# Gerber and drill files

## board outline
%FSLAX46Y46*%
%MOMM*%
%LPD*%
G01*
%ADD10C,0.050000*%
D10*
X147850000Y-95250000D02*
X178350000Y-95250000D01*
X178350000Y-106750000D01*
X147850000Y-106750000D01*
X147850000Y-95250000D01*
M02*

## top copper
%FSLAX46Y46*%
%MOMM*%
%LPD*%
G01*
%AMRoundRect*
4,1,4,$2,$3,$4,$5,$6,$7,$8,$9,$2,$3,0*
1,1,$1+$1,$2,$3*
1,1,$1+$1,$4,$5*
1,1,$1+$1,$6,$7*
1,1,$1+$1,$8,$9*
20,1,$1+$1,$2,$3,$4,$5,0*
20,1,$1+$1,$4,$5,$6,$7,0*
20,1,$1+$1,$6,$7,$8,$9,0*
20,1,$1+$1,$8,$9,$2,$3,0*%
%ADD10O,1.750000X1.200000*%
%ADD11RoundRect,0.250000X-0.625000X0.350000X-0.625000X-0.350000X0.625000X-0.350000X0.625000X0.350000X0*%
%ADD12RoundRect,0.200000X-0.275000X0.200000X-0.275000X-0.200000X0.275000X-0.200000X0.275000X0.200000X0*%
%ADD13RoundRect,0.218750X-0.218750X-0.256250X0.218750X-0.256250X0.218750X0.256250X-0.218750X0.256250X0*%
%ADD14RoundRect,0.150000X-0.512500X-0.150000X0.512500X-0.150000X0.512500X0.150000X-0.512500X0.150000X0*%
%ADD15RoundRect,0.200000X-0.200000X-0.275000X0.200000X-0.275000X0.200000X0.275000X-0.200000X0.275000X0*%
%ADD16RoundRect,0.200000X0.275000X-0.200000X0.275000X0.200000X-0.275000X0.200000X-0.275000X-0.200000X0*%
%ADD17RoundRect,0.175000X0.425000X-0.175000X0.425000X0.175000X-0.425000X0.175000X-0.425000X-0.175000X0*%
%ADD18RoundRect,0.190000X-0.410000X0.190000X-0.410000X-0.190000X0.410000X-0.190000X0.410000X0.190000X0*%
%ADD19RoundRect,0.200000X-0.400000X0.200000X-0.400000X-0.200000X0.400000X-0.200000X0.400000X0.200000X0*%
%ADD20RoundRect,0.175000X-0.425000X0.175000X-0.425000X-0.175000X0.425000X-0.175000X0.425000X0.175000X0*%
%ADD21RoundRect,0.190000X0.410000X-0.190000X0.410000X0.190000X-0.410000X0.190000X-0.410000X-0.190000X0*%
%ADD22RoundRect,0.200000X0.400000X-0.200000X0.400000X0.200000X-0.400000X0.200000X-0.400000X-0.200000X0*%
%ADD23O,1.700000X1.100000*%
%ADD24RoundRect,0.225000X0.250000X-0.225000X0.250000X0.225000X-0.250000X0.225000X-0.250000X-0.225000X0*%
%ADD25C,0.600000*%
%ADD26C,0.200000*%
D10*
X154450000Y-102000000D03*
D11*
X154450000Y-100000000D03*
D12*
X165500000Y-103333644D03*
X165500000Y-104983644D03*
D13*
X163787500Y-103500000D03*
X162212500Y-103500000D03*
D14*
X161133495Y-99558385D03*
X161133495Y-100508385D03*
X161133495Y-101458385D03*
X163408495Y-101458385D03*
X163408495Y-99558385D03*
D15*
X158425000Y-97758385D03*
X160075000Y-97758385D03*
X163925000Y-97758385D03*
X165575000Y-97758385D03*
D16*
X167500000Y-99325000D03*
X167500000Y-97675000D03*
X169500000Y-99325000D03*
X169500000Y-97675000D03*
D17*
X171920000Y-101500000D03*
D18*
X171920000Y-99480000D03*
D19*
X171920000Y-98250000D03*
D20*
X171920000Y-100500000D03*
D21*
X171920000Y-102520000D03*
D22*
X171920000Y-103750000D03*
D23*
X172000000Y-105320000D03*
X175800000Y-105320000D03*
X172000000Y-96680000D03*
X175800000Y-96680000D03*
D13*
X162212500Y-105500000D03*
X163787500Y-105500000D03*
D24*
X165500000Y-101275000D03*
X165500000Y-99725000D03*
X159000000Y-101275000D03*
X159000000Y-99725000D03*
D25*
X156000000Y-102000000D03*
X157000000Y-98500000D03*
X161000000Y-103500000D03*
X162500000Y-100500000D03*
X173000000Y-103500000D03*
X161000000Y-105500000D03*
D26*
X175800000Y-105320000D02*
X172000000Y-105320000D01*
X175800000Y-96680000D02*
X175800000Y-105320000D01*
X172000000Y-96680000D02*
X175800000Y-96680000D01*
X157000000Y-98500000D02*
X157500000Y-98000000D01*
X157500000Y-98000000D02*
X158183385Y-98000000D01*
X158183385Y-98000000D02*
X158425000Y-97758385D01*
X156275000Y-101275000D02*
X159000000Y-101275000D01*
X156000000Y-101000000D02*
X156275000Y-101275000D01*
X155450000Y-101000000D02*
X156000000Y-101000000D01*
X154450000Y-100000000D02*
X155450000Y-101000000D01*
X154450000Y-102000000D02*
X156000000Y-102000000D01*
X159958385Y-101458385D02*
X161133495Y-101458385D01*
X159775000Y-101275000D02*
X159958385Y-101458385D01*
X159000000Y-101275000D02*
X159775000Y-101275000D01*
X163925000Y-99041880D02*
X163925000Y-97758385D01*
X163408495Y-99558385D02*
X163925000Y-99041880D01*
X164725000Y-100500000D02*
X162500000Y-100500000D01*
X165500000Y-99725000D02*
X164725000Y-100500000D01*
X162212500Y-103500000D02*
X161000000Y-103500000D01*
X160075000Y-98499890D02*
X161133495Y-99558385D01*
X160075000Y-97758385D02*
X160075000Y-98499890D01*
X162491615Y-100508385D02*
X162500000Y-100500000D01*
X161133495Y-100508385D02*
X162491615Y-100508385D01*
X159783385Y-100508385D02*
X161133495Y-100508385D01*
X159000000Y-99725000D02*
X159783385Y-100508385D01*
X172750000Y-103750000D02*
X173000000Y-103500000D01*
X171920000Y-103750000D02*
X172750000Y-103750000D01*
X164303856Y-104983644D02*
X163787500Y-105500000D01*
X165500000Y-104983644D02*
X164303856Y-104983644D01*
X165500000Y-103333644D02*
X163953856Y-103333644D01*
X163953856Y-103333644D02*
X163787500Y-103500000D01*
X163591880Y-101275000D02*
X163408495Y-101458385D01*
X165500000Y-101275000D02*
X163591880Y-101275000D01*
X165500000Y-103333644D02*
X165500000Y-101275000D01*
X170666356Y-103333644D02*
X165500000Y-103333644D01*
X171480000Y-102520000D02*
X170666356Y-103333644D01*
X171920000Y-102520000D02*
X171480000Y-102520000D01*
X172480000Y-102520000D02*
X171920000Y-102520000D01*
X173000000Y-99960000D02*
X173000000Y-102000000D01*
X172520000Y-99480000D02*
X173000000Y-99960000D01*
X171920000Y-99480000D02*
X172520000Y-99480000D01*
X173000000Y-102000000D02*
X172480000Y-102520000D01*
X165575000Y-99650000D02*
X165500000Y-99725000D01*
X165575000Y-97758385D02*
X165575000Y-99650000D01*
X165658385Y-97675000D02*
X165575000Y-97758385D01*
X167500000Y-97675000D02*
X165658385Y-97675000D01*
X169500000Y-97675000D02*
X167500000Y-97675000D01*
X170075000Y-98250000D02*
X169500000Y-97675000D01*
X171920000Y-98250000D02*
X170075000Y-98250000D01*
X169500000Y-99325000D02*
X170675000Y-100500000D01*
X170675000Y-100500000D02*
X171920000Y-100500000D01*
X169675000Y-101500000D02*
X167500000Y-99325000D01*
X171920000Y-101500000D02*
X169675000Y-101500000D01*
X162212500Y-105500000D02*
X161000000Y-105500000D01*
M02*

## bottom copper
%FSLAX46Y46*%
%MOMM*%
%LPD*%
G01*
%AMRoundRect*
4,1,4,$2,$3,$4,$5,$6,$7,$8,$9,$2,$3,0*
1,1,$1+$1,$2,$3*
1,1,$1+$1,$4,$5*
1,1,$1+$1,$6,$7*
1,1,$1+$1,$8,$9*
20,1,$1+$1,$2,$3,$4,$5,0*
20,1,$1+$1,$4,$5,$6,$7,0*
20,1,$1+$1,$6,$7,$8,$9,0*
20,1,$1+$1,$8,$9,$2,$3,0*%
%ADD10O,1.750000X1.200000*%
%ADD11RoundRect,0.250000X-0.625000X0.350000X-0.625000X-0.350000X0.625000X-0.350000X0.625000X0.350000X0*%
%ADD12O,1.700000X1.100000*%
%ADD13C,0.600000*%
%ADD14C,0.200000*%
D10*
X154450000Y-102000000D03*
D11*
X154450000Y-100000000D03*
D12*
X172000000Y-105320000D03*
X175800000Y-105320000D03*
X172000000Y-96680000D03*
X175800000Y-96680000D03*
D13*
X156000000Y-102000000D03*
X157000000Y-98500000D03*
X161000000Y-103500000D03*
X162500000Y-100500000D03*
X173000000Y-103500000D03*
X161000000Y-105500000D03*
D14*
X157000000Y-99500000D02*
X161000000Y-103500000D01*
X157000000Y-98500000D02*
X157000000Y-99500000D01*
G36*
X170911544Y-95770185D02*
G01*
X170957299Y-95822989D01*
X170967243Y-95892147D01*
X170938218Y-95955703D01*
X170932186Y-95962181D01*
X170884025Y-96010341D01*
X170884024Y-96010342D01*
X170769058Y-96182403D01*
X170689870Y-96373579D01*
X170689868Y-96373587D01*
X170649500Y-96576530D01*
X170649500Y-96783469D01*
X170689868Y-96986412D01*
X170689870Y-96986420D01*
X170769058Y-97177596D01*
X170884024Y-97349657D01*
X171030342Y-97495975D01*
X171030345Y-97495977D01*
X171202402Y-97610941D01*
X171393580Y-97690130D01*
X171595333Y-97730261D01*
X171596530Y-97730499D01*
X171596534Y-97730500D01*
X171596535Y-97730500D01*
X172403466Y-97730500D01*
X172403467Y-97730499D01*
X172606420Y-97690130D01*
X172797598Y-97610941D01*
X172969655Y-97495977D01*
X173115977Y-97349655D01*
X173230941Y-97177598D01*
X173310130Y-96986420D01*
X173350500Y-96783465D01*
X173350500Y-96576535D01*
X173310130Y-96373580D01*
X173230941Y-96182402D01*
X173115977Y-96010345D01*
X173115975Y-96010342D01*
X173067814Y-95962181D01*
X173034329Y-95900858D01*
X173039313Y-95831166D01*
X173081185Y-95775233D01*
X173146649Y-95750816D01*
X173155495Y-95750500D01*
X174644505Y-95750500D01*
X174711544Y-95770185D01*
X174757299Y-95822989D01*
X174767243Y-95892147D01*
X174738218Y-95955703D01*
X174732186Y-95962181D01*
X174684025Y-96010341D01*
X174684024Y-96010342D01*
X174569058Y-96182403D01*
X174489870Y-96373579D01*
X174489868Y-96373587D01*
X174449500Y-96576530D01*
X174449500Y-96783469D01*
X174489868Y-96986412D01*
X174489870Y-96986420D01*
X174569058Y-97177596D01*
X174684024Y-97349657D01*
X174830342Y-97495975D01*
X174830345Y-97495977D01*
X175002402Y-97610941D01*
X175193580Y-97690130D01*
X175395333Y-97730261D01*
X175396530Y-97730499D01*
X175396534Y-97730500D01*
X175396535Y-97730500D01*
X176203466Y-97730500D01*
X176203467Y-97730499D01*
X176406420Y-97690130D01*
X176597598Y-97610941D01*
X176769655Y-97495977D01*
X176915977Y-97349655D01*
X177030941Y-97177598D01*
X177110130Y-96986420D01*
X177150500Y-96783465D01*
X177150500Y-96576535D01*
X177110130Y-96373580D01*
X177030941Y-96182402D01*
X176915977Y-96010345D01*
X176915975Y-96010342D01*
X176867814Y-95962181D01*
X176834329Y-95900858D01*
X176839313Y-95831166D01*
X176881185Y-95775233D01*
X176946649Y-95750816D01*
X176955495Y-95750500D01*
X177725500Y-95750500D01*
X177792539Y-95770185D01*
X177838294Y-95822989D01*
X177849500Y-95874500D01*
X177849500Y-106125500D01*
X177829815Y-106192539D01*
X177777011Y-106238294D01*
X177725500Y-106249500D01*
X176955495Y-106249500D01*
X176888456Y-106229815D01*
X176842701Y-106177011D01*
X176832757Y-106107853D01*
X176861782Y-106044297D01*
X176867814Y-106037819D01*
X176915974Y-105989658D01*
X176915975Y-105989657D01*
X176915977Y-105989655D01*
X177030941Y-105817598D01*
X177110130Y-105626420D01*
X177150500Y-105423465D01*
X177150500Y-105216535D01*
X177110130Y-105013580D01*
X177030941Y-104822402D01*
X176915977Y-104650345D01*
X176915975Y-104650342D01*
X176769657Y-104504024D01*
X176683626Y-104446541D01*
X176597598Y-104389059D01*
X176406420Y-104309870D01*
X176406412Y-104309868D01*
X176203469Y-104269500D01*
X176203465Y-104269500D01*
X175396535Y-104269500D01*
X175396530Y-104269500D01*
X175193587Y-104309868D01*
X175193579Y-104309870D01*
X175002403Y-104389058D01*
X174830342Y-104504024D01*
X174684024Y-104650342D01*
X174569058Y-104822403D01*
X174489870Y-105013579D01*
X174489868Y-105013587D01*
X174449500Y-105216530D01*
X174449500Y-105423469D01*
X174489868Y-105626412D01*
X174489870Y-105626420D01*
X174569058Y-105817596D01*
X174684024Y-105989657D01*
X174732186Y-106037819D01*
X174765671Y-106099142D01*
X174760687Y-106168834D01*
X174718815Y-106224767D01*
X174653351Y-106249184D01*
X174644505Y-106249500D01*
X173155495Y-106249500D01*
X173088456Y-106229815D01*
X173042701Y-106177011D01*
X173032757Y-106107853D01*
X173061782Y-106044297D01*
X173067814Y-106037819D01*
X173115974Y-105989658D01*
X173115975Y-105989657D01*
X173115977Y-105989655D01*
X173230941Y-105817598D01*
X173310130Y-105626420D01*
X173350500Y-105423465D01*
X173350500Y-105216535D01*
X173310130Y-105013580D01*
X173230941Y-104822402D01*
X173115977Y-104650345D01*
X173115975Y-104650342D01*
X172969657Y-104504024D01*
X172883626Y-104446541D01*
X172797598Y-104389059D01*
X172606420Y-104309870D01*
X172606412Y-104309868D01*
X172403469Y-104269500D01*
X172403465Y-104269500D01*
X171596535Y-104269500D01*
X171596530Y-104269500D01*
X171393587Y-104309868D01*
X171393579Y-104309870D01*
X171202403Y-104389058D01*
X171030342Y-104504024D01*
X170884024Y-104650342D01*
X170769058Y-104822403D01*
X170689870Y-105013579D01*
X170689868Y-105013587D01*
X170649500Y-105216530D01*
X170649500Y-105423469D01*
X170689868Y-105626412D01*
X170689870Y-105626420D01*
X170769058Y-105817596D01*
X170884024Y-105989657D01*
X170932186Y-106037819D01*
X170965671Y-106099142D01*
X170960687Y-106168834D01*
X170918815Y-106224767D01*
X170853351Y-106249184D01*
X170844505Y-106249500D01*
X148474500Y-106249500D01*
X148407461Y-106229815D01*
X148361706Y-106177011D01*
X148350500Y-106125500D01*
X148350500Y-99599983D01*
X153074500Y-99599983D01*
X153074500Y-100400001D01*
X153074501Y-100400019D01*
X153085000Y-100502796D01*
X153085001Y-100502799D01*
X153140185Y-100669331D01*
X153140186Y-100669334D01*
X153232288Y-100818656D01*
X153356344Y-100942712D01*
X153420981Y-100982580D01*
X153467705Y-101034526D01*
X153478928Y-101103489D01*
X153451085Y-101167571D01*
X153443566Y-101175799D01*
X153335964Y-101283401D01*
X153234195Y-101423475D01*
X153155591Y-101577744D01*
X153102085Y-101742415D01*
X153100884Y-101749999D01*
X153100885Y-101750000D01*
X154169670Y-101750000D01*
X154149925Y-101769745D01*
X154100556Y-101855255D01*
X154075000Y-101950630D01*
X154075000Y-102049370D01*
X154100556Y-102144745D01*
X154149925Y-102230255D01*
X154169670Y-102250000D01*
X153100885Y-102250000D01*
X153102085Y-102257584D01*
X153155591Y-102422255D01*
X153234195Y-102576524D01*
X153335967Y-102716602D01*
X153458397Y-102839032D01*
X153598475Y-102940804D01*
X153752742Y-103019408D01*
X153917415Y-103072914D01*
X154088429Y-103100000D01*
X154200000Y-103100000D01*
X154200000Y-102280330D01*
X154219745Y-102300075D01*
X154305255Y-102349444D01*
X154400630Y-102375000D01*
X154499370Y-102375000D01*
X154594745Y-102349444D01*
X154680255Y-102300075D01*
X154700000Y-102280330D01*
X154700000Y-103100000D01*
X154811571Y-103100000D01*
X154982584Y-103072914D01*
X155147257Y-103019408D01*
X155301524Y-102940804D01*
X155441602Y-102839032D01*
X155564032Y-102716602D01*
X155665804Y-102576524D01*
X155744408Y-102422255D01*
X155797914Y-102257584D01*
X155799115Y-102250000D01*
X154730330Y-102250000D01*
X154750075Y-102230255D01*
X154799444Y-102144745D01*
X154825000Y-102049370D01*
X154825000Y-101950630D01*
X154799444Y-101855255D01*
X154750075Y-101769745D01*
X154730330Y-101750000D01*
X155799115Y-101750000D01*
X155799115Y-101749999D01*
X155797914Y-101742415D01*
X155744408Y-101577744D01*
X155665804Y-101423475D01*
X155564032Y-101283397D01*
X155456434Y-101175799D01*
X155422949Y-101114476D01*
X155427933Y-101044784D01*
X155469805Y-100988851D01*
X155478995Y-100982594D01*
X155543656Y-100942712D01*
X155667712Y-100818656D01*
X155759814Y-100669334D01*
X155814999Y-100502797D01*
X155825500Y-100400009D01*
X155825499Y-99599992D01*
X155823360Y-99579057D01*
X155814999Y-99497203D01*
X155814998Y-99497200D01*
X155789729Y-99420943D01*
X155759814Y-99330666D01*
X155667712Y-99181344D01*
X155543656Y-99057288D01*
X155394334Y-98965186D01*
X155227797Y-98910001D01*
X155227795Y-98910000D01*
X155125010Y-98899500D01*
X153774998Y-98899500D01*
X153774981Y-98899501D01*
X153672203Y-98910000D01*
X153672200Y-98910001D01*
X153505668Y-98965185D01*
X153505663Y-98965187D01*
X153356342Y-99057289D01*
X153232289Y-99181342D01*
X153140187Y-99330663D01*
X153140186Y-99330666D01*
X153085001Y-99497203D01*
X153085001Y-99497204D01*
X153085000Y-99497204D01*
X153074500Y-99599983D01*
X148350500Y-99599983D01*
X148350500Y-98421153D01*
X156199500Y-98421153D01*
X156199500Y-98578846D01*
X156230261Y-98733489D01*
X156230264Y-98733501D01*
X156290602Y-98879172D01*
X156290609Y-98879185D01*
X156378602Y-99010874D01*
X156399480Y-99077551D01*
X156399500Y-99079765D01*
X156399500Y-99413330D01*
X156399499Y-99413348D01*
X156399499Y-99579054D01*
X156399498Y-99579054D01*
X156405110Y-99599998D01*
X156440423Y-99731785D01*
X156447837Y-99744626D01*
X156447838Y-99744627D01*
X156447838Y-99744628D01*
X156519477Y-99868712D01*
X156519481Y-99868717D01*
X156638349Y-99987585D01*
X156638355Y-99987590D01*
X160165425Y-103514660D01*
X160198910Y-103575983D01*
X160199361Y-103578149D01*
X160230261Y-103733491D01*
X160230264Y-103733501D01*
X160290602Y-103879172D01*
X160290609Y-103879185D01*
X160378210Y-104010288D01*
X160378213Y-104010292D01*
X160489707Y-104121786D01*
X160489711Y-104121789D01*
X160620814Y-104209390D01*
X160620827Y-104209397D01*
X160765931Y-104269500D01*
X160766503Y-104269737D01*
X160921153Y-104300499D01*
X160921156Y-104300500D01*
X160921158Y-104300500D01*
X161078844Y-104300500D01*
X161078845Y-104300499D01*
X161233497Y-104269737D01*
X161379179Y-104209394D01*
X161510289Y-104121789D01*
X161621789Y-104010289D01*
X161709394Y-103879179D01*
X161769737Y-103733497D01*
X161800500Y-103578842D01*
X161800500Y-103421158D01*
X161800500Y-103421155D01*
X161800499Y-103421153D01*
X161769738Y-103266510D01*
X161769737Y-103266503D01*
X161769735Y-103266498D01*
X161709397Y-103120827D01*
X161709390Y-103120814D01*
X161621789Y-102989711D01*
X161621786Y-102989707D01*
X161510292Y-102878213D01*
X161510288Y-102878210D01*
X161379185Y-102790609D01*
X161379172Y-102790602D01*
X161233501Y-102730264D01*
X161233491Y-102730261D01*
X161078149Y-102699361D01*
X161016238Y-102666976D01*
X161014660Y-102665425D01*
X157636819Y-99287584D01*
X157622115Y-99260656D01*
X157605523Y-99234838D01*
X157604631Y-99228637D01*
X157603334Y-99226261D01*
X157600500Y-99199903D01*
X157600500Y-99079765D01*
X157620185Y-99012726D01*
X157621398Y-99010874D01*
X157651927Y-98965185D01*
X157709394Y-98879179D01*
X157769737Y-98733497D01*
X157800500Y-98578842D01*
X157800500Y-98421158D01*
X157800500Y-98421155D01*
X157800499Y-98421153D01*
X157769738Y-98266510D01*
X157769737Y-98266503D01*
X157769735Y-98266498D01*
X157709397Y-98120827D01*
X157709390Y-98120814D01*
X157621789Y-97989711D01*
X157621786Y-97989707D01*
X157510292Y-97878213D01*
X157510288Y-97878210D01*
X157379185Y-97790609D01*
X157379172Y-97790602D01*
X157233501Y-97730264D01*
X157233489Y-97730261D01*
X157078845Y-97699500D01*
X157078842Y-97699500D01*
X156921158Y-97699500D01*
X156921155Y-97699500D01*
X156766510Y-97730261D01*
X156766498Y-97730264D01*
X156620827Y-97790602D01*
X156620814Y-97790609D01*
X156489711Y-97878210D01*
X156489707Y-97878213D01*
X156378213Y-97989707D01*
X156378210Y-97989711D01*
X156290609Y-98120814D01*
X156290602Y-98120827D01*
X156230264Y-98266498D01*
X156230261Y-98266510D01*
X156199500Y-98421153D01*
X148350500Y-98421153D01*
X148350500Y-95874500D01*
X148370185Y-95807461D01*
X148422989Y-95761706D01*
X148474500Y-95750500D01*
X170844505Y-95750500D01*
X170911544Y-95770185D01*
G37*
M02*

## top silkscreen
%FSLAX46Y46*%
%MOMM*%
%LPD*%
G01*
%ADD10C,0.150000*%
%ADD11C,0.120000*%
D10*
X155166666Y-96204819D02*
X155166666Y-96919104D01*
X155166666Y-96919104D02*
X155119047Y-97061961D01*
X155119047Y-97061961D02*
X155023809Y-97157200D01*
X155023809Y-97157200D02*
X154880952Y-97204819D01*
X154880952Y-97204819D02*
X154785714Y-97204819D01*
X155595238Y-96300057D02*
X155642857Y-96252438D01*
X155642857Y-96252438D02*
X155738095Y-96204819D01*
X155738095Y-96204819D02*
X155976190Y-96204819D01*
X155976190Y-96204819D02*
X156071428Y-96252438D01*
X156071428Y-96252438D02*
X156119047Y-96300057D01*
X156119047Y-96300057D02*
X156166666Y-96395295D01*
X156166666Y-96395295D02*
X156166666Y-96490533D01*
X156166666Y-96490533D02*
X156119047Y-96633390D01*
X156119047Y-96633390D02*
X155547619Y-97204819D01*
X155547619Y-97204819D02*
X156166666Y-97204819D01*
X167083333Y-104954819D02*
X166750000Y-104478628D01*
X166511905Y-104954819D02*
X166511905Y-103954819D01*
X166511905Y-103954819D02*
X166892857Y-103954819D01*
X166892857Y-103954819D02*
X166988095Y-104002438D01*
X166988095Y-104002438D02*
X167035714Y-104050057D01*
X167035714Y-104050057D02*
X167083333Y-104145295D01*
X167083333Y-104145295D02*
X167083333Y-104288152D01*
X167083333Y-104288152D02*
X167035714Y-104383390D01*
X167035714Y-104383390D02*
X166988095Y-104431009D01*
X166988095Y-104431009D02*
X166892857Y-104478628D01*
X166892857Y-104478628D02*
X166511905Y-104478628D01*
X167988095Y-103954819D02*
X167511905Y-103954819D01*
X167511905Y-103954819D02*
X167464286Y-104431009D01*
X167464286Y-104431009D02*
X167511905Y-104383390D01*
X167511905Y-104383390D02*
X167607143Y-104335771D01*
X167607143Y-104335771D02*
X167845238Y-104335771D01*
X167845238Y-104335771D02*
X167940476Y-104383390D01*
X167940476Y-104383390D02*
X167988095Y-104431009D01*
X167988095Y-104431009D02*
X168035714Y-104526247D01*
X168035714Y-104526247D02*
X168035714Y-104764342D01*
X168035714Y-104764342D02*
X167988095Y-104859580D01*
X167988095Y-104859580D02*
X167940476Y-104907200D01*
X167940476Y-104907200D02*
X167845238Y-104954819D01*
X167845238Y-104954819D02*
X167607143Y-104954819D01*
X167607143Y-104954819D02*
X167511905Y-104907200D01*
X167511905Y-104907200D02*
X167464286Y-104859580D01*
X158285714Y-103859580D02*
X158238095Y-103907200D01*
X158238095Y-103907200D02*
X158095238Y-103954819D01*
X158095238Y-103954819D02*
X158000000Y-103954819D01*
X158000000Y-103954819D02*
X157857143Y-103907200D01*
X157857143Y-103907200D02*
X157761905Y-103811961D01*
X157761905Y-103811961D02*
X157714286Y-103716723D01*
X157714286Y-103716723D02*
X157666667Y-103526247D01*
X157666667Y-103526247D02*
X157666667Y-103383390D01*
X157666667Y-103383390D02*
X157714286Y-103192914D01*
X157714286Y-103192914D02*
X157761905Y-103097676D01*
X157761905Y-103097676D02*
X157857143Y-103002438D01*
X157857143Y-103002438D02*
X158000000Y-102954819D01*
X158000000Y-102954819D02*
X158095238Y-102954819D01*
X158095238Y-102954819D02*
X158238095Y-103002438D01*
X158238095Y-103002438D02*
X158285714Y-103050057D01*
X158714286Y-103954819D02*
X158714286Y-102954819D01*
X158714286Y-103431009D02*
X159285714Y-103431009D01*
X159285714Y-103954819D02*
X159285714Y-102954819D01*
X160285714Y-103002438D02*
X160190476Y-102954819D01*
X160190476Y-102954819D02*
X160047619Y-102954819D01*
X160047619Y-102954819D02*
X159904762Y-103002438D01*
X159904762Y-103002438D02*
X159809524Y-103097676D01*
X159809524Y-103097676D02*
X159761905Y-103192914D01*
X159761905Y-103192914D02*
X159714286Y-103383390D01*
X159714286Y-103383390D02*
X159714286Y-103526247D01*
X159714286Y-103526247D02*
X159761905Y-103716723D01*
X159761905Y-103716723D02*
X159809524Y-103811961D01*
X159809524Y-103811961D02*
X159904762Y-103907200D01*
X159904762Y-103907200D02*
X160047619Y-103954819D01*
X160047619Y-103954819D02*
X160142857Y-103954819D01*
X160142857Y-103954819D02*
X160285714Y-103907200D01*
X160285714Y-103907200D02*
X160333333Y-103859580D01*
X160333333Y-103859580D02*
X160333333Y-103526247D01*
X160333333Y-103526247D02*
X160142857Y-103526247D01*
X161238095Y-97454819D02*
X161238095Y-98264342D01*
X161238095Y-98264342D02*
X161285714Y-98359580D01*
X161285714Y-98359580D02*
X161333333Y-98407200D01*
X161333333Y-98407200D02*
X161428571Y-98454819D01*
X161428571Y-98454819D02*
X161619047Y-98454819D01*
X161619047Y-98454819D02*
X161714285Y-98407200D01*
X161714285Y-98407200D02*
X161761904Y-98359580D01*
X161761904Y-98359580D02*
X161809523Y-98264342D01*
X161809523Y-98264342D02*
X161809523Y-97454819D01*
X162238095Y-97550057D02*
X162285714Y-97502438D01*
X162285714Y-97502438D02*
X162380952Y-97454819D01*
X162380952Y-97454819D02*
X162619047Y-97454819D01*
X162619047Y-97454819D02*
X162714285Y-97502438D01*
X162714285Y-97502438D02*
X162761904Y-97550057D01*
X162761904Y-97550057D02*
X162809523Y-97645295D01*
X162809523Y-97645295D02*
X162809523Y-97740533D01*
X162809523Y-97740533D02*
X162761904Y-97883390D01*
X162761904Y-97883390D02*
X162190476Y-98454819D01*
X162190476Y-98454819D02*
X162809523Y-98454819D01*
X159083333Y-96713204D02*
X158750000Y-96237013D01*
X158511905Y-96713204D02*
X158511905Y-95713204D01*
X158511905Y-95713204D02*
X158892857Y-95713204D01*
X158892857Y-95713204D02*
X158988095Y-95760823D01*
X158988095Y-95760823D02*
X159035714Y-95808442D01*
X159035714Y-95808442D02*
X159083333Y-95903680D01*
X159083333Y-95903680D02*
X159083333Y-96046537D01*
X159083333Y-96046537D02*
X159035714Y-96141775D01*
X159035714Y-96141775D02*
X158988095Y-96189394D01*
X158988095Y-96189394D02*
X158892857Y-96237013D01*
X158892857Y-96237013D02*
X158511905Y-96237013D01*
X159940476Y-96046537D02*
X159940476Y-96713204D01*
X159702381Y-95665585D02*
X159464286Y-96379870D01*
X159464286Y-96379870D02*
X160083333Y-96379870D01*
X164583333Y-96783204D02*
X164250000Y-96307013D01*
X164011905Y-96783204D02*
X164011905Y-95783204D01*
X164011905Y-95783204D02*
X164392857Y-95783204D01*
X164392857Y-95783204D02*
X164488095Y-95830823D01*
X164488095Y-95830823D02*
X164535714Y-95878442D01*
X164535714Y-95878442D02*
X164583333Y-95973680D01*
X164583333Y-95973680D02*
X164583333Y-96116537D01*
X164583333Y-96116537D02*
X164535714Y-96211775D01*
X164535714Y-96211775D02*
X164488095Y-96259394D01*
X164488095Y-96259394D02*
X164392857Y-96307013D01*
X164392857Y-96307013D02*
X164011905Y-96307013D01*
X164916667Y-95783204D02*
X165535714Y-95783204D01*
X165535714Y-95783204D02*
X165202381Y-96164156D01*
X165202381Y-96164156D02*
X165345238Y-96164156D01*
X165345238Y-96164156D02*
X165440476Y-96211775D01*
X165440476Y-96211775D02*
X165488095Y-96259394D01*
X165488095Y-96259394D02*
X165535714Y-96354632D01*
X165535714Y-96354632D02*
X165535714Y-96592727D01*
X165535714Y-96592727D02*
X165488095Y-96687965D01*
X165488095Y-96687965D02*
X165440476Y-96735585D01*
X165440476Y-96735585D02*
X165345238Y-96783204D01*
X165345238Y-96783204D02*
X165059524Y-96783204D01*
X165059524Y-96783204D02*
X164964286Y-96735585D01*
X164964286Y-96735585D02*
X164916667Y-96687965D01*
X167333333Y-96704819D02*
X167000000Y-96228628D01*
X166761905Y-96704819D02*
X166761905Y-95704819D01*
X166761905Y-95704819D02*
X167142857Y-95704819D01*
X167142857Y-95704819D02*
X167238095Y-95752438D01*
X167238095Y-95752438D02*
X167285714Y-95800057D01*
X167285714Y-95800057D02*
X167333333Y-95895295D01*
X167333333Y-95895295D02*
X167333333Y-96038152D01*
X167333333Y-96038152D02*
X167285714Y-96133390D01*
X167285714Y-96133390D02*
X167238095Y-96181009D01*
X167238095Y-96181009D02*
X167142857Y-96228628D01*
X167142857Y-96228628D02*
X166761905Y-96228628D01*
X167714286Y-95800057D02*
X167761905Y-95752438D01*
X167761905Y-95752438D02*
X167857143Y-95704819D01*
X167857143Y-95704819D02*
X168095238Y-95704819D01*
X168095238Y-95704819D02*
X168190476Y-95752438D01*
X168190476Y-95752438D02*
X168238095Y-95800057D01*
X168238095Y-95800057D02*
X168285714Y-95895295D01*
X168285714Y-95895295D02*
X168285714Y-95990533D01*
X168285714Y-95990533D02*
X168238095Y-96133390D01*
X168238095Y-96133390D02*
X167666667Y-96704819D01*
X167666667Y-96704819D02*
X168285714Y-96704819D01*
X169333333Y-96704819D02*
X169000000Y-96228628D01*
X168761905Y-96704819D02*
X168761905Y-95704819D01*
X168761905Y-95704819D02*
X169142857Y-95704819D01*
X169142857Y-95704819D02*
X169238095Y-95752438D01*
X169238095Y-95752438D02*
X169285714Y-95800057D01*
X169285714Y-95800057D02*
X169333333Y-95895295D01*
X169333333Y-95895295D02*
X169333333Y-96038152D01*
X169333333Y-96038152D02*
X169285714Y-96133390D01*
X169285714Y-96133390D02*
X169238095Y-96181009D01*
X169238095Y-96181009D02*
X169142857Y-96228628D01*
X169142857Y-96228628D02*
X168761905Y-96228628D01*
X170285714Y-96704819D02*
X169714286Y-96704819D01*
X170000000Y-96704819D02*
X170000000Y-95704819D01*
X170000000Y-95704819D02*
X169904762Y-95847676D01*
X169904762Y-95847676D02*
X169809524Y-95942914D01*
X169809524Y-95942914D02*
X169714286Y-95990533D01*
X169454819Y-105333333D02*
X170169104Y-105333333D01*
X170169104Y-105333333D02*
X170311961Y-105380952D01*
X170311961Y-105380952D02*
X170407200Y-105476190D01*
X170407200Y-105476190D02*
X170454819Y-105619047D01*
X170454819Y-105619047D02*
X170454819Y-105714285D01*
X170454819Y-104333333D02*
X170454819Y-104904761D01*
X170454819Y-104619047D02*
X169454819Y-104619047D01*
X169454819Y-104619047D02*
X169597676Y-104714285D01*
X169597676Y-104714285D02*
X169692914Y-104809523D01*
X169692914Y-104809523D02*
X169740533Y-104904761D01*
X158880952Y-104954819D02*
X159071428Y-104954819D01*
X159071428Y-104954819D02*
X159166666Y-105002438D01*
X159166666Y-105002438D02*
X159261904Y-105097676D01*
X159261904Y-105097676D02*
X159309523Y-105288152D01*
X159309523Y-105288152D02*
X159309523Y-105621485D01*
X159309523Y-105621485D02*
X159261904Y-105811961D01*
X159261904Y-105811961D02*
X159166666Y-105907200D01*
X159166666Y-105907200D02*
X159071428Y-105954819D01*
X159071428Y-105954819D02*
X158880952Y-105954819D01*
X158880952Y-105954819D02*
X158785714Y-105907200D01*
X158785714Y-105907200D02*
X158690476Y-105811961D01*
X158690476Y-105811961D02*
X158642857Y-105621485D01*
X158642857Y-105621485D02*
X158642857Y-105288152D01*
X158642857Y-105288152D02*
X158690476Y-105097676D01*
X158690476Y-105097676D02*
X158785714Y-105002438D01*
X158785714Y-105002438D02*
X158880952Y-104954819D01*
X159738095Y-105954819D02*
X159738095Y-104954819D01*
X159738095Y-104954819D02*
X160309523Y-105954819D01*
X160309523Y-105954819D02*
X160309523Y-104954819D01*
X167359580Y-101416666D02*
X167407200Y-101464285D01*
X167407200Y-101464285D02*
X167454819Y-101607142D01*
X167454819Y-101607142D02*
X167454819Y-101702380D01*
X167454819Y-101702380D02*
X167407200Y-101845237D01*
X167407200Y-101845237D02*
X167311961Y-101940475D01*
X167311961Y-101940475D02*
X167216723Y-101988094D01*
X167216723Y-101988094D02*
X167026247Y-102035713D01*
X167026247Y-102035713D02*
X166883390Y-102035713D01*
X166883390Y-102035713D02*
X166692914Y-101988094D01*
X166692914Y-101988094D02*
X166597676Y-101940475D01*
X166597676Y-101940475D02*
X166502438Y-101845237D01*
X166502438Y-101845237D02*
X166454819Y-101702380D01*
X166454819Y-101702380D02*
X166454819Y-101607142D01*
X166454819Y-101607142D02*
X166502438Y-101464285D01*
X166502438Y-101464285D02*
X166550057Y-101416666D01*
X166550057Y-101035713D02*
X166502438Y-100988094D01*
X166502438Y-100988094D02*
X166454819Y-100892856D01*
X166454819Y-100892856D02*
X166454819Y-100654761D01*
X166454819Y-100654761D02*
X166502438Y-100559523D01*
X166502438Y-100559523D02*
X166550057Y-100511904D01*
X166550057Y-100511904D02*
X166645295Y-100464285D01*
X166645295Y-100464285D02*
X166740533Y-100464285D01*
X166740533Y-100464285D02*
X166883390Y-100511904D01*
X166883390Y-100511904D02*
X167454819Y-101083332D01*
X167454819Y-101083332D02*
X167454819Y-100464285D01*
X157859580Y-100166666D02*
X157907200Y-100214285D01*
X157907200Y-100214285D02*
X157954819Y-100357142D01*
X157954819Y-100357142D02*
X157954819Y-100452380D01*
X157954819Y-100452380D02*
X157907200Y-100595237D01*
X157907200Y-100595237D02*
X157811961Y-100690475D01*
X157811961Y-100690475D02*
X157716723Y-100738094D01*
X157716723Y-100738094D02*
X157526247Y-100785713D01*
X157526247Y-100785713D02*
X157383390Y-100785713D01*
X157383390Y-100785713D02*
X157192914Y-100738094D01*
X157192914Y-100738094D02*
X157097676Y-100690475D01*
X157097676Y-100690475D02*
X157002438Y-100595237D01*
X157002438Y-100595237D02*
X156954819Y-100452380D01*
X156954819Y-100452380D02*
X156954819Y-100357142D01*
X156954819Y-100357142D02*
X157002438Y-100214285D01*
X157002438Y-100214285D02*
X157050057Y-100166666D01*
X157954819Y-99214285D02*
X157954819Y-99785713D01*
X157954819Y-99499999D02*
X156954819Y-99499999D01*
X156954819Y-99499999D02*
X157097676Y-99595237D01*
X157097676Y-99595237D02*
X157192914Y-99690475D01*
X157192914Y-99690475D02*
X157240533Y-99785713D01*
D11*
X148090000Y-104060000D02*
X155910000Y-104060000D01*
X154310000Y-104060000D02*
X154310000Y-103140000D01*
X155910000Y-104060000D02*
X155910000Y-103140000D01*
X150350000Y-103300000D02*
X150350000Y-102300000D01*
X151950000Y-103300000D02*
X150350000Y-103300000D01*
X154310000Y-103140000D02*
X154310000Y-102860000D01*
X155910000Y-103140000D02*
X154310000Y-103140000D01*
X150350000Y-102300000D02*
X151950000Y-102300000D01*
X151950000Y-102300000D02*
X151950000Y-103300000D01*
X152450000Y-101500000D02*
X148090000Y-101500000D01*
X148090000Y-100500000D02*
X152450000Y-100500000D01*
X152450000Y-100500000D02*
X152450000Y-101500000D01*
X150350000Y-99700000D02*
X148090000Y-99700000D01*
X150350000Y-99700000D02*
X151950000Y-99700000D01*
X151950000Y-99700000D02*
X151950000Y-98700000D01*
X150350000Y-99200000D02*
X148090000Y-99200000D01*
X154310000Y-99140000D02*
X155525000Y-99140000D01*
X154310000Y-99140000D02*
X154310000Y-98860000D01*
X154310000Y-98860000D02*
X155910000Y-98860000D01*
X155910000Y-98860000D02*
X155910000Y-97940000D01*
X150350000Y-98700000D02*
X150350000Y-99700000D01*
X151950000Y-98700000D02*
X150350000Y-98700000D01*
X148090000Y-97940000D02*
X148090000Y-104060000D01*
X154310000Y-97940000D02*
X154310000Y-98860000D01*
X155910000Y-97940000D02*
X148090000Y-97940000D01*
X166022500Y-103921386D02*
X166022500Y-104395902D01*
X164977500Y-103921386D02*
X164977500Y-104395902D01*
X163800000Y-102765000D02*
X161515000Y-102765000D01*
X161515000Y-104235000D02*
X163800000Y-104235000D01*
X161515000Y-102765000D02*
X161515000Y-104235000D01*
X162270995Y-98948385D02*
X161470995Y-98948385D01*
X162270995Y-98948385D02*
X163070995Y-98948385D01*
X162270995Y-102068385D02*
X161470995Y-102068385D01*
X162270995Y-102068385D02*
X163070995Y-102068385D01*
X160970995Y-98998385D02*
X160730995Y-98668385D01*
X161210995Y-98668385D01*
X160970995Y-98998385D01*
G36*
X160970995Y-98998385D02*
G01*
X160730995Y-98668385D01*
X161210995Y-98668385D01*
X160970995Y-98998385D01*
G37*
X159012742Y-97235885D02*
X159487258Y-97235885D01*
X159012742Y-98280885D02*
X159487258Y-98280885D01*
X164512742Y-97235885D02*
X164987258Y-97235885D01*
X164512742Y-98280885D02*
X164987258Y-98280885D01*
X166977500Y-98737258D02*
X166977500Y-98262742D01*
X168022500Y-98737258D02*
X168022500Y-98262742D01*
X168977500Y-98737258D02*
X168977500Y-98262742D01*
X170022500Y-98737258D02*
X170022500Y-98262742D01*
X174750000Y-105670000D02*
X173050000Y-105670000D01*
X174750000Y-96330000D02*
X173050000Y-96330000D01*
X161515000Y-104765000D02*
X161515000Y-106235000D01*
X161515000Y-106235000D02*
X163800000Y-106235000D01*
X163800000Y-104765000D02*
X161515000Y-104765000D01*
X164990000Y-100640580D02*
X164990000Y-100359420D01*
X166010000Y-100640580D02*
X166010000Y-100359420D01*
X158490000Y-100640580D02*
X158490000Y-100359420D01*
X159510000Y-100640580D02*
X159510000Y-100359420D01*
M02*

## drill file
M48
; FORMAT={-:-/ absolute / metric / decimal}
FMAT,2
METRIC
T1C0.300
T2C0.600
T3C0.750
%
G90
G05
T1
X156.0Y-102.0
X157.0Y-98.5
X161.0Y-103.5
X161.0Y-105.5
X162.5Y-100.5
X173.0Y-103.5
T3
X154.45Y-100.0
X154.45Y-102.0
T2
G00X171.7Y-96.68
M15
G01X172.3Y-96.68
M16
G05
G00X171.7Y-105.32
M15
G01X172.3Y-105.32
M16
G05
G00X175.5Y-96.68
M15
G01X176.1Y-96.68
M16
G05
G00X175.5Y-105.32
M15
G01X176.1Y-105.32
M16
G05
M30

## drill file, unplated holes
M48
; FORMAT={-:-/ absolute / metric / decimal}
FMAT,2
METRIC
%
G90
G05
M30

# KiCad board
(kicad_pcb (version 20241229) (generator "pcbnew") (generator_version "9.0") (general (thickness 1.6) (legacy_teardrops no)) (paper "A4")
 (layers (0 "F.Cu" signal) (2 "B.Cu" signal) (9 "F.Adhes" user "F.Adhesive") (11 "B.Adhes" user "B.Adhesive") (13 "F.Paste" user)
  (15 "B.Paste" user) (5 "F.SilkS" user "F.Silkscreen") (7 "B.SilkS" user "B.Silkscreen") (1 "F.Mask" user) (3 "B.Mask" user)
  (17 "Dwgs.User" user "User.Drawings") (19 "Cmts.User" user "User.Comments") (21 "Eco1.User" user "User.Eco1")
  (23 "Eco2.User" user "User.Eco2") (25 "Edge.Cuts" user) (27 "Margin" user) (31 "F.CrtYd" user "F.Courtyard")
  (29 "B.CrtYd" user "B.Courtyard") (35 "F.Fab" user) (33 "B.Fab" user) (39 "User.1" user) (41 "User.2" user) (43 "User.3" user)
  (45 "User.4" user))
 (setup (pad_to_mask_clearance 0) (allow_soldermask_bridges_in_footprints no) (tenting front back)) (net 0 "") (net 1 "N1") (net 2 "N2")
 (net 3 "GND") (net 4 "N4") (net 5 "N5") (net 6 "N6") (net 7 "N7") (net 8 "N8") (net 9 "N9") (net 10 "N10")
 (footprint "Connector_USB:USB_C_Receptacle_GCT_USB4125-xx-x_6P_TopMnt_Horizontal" (layer "F.Cu") (at 175 101 90)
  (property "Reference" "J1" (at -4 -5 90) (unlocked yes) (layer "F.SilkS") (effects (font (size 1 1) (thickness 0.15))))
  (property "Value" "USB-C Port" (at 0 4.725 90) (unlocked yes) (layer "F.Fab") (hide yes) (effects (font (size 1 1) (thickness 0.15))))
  (fp_line (start 4.67 -0.25) (end 4.67 -1.95) (stroke (width 0.12) (type solid)) (layer "F.SilkS"))
  (fp_line (start -4.67 -0.25) (end -4.67 -1.95) (stroke (width 0.12) (type solid)) (layer "F.SilkS"))
  (pad "A5" smd roundrect (at -0.5 -3.08 90) (size 0.7 1.2) (layers "F.Cu" "F.Mask" "F.Paste") (roundrect_rratio 0.25) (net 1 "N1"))
  (pad "A9" smd roundrect (at 1.52 -3.08 270) (size 0.76 1.2) (layers "F.Cu" "F.Mask" "F.Paste") (roundrect_rratio 0.25) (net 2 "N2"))
  (pad "A12" smd roundrect (at 2.75 -3.08 270) (size 0.8 1.2) (layers "F.Cu" "F.Mask" "F.Paste") (roundrect_rratio 0.25) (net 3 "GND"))
  (pad "B5" smd roundrect (at 0.5 -3.08 270) (size 0.7 1.2) (layers "F.Cu" "F.Mask" "F.Paste") (roundrect_rratio 0.25) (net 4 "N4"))
  (pad "B9" smd roundrect (at -1.52 -3.08 90) (size 0.76 1.2) (layers "F.Cu" "F.Mask" "F.Paste") (roundrect_rratio 0.25) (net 2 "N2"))
  (pad "B12" smd roundrect (at -2.75 -3.08 90) (size 0.8 1.2) (layers "F.Cu" "F.Mask" "F.Paste") (roundrect_rratio 0.25) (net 3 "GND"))
  (pad "S1" thru_hole oval (at -4.32 -3 90) (size 1.1 1.7) (drill oval 0.6 1.2) (layers "*.Cu" "*.Mask" "F.Paste") (remove_unused_layers no)
   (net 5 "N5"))
  (pad "S1" thru_hole oval (at -4.32 0.8 90) (size 1.1 1.7) (drill oval 0.6 1.2) (layers "*.Cu" "*.Mask" "F.Paste")
   (remove_unused_layers no) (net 5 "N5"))
  (pad "S1" thru_hole oval (at 4.32 -3 90) (size 1.1 1.7) (drill oval 0.6 1.2) (layers "*.Cu" "*.Mask" "F.Paste") (remove_unused_layers no)
   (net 5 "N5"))
  (pad "S1" thru_hole oval (at 4.32 0.8 90) (size 1.1 1.7) (drill oval 0.6 1.2) (layers "*.Cu" "*.Mask" "F.Paste") (remove_unused_layers no)
   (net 5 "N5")))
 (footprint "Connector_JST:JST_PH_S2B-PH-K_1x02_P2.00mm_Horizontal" (layer "F.Cu") (at 154.45 100 -90)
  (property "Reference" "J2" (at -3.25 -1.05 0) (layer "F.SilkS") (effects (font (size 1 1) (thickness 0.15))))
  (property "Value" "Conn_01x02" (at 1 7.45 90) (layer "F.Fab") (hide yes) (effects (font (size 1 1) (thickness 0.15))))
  (fp_line (start -2.06 6.36) (end 4.06 6.36) (stroke (width 0.12) (type solid)) (layer "F.SilkS"))
  (fp_line (start 0.5 6.36) (end 0.5 2) (stroke (width 0.12) (type solid)) (layer "F.SilkS"))
  (fp_line (start 4.06 6.36) (end 4.06 -1.46) (stroke (width 0.12) (type solid)) (layer "F.SilkS"))
  (fp_line (start -1.3 4.1) (end -0.3 4.1) (stroke (width 0.12) (type solid)) (layer "F.SilkS"))
  (fp_line (start -0.8 4.1) (end -0.8 6.36) (stroke (width 0.12) (type solid)) (layer "F.SilkS"))
  (fp_line (start -0.3 4.1) (end -0.3 6.36) (stroke (width 0.12) (type solid)) (layer "F.SilkS"))
  (fp_line (start -0.3 4.1) (end -0.3 2.5) (stroke (width 0.12) (type solid)) (layer "F.SilkS"))
  (fp_line (start 2.3 4.1) (end 2.3 2.5) (stroke (width 0.12) (type solid)) (layer "F.SilkS"))
  (fp_line (start 3.3 4.1) (end 2.3 4.1) (stroke (width 0.12) (type solid)) (layer "F.SilkS"))
  (fp_line (start -1.3 2.5) (end -1.3 4.1) (stroke (width 0.12) (type solid)) (layer "F.SilkS"))
  (fp_line (start -0.3 2.5) (end -1.3 2.5) (stroke (width 0.12) (type solid)) (layer "F.SilkS"))
  (fp_line (start 2.3 2.5) (end 3.3 2.5) (stroke (width 0.12) (type solid)) (layer "F.SilkS"))
  (fp_line (start 3.3 2.5) (end 3.3 4.1) (stroke (width 0.12) (type solid)) (layer "F.SilkS"))
  (fp_line (start 0.5 2) (end 1.5 2) (stroke (width 0.12) (type solid)) (layer "F.SilkS"))
  (fp_line (start 1.5 2) (end 1.5 6.36) (stroke (width 0.12) (type solid)) (layer "F.SilkS"))
  (fp_line (start -2.06 0.14) (end -1.14 0.14) (stroke (width 0.12) (type solid)) (layer "F.SilkS"))
  (fp_line (start -1.14 0.14) (end -1.14 -1.46) (stroke (width 0.12) (type solid)) (layer "F.SilkS"))
  (fp_line (start -0.86 0.14) (end -1.14 0.14) (stroke (width 0.12) (type solid)) (layer "F.SilkS"))
  (fp_line (start -0.86 0.14) (end -0.86 -1.075) (stroke (width 0.12) (type solid)) (layer "F.SilkS"))
  (fp_line (start 3.14 0.14) (end 2.86 0.14) (stroke (width 0.12) (type solid)) (layer "F.SilkS"))
  (fp_line (start 4.06 0.14) (end 3.14 0.14) (stroke (width 0.12) (type solid)) (layer "F.SilkS"))
  (fp_line (start -2.06 -1.46) (end -2.06 6.36) (stroke (width 0.12) (type solid)) (layer "F.SilkS"))
  (fp_line (start -1.14 -1.46) (end -2.06 -1.46) (stroke (width 0.12) (type solid)) (layer "F.SilkS"))
  (fp_line (start 3.14 -1.46) (end 3.14 0.14) (stroke (width 0.12) (type solid)) (layer "F.SilkS"))
  (fp_line (start 4.06 -1.46) (end 3.14 -1.46) (stroke (width 0.12) (type solid)) (layer "F.SilkS"))
  (pad "1" thru_hole roundrect (at 0 0 270) (size 1.2 1.75) (drill 0.75) (layers "*.Cu" "*.Mask") (remove_unused_layers no)
   (roundrect_rratio 0.208333) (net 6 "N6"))
  (pad "2" thru_hole oval (at 2 0 270) (size 1.2 1.75) (drill 0.75) (layers "*.Cu" "*.Mask") (remove_unused_layers no) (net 3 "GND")))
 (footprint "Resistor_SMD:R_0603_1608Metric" (layer "F.Cu") (at 164.75 97.758385)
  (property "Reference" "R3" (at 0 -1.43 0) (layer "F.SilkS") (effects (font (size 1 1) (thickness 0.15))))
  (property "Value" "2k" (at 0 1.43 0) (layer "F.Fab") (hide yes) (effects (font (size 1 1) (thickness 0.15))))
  (fp_line (start -0.237258 -0.5225) (end 0.237258 -0.5225) (stroke (width 0.12) (type solid)) (layer "F.SilkS"))
  (fp_line (start -0.237258 0.5225) (end 0.237258 0.5225) (stroke (width 0.12) (type solid)) (layer "F.SilkS"))
  (pad "1" smd roundrect (at -0.825 0) (size 0.8 0.95) (layers "F.Cu" "F.Mask" "F.Paste") (roundrect_rratio 0.25) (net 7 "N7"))
  (pad "2" smd roundrect (at 0.825 0) (size 0.8 0.95) (layers "F.Cu" "F.Mask" "F.Paste") (roundrect_rratio 0.25) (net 3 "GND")))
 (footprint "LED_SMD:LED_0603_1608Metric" (layer "F.Cu") (at 163 103.5)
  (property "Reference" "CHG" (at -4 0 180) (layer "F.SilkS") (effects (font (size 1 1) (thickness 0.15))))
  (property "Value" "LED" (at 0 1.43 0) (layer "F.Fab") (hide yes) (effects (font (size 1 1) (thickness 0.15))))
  (fp_line (start -1.485 -0.735) (end -1.485 0.735) (stroke (width 0.12) (type solid)) (layer "F.SilkS"))
  (fp_line (start -1.485 0.735) (end 0.8 0.735) (stroke (width 0.12) (type solid)) (layer "F.SilkS"))
  (fp_line (start 0.8 -0.735) (end -1.485 -0.735) (stroke (width 0.12) (type solid)) (layer "F.SilkS"))
  (pad "1" smd roundrect (at -0.7875 0) (size 0.875 0.95) (layers "F.Cu" "F.Mask" "F.Paste") (roundrect_rratio 0.25) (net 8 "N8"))
  (pad "2" smd roundrect (at 0.7875 0) (size 0.875 0.95) (layers "F.Cu" "F.Mask" "F.Paste") (roundrect_rratio 0.25) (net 2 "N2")))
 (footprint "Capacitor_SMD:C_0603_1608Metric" (layer "F.Cu") (at 165.5 100.5 90)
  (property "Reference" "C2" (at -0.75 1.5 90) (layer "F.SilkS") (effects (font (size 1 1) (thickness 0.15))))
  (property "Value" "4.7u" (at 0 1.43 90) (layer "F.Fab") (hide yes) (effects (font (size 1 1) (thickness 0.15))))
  (fp_line (start -0.14058 -0.51) (end 0.14058 -0.51) (stroke (width 0.12) (type solid)) (layer "F.SilkS"))
  (fp_line (start -0.14058 0.51) (end 0.14058 0.51) (stroke (width 0.12) (type solid)) (layer "F.SilkS"))
  (pad "1" smd roundrect (at -0.775 0 90) (size 0.9 0.95) (layers "F.Cu" "F.Mask" "F.Paste") (roundrect_rratio 0.25) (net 2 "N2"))
  (pad "2" smd roundrect (at 0.775 0 90) (size 0.9 0.95) (layers "F.Cu" "F.Mask" "F.Paste") (roundrect_rratio 0.25) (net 3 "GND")))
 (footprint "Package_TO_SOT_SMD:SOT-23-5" (layer "F.Cu") (at 162.270995 100.508385)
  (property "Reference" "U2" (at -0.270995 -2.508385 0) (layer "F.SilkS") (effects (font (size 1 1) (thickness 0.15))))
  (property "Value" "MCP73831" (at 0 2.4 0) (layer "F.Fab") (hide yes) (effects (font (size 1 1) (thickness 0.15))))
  (fp_line (start 0 -1.56) (end -0.8 -1.56) (stroke (width 0.12) (type solid)) (layer "F.SilkS"))
  (fp_line (start 0 -1.56) (end 0.8 -1.56) (stroke (width 0.12) (type solid)) (layer "F.SilkS"))
  (fp_line (start 0 1.56) (end -0.8 1.56) (stroke (width 0.12) (type solid)) (layer "F.SilkS"))
  (fp_line (start 0 1.56) (end 0.8 1.56) (stroke (width 0.12) (type solid)) (layer "F.SilkS"))
  (fp_poly
   (pts (xy -1.3 -1.51) (xy -1.54 -1.84) (xy -1.06 -1.84) (xy -1.3 -1.51)) (stroke (width 0.12) (type solid)) (fill yes) (layer "F.SilkS"))
  (pad "1" smd roundrect (at -1.1375 -0.95) (size 1.325 0.6) (layers "F.Cu" "F.Mask" "F.Paste") (roundrect_rratio 0.25) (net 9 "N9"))
  (pad "2" smd roundrect (at -1.1375 0) (size 1.325 0.6) (layers "F.Cu" "F.Mask" "F.Paste") (roundrect_rratio 0.25) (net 3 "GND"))
  (pad "3" smd roundrect (at -1.1375 0.95) (size 1.325 0.6) (layers "F.Cu" "F.Mask" "F.Paste") (roundrect_rratio 0.25) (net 6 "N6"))
  (pad "4" smd roundrect (at 1.1375 0.95) (size 1.325 0.6) (layers "F.Cu" "F.Mask" "F.Paste") (roundrect_rratio 0.25) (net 2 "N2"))
  (pad "5" smd roundrect (at 1.1375 -0.95) (size 1.325 0.6) (layers "F.Cu" "F.Mask" "F.Paste") (roundrect_rratio 0.25) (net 7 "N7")))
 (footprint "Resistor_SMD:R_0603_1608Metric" (layer "F.Cu") (at 167.5 98.5 90)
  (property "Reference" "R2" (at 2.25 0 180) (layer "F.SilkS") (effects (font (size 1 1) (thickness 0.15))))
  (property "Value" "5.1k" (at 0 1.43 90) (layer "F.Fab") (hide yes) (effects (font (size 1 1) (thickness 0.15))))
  (fp_line (start -0.237258 -0.5225) (end 0.237258 -0.5225) (stroke (width 0.12) (type solid)) (layer "F.SilkS"))
  (fp_line (start -0.237258 0.5225) (end 0.237258 0.5225) (stroke (width 0.12) (type solid)) (layer "F.SilkS"))
  (pad "1" smd roundrect (at -0.825 0 90) (size 0.8 0.95) (layers "F.Cu" "F.Mask" "F.Paste") (roundrect_rratio 0.25) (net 1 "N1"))
  (pad "2" smd roundrect (at 0.825 0 90) (size 0.8 0.95) (layers "F.Cu" "F.Mask" "F.Paste") (roundrect_rratio 0.25) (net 3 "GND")))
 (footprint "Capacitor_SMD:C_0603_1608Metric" (layer "F.Cu") (at 159 100.5 90)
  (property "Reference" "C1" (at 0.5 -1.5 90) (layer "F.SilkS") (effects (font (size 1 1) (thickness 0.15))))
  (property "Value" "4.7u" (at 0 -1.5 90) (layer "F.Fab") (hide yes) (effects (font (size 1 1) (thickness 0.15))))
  (fp_line (start -0.14058 -0.51) (end 0.14058 -0.51) (stroke (width 0.12) (type solid)) (layer "F.SilkS"))
  (fp_line (start -0.14058 0.51) (end 0.14058 0.51) (stroke (width 0.12) (type solid)) (layer "F.SilkS"))
  (pad "1" smd roundrect (at -0.775 0 90) (size 0.9 0.95) (layers "F.Cu" "F.Mask" "F.Paste") (roundrect_rratio 0.25) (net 6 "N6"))
  (pad "2" smd roundrect (at 0.775 0 90) (size 0.9 0.95) (layers "F.Cu" "F.Mask" "F.Paste") (roundrect_rratio 0.25) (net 3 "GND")))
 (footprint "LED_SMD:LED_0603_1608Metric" (layer "F.Cu") (at 163 105.5)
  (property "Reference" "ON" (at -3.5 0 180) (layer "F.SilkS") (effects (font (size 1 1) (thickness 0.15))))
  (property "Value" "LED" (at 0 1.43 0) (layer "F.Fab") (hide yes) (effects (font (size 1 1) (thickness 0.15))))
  (fp_line (start -1.485 -0.735) (end -1.485 0.735) (stroke (width 0.12) (type solid)) (layer "F.SilkS"))
  (fp_line (start -1.485 0.735) (end 0.8 0.735) (stroke (width 0.12) (type solid)) (layer "F.SilkS"))
  (fp_line (start 0.8 -0.735) (end -1.485 -0.735) (stroke (width 0.12) (type solid)) (layer "F.SilkS"))
  (pad "1" smd roundrect (at -0.7875 0) (size 0.875 0.95) (layers "F.Cu" "F.Mask" "F.Paste") (roundrect_rratio 0.25) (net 3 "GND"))
  (pad "2" smd roundrect (at 0.7875 0) (size 0.875 0.95) (layers "F.Cu" "F.Mask" "F.Paste") (roundrect_rratio 0.25) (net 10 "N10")))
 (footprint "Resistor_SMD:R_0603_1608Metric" (layer "F.Cu") (at 165.5 104.158644 -90)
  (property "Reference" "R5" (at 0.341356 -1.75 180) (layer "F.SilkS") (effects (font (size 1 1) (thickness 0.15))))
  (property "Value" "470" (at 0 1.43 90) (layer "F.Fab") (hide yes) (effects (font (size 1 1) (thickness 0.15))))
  (fp_line (start -0.237258 0.5225) (end 0.237258 0.5225) (stroke (width 0.12) (type solid)) (layer "F.SilkS"))
  (fp_line (start -0.237258 -0.5225) (end 0.237258 -0.5225) (stroke (width 0.12) (type solid)) (layer "F.SilkS"))
  (pad "1" smd roundrect (at -0.825 0 270) (size 0.8 0.95) (layers "F.Cu" "F.Mask" "F.Paste") (roundrect_rratio 0.25) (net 2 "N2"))
  (pad "2" smd roundrect (at 0.825 0 270) (size 0.8 0.95) (layers "F.Cu" "F.Mask" "F.Paste") (roundrect_rratio 0.25) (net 10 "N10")))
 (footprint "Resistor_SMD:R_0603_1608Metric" (layer "F.Cu") (at 169.5 98.5 90)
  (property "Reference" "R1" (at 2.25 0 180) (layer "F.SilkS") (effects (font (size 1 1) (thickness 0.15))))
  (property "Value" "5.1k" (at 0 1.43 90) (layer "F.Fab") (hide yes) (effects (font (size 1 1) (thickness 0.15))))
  (fp_line (start -0.237258 -0.5225) (end 0.237258 -0.5225) (stroke (width 0.12) (type solid)) (layer "F.SilkS"))
  (fp_line (start -0.237258 0.5225) (end 0.237258 0.5225) (stroke (width 0.12) (type solid)) (layer "F.SilkS"))
  (pad "1" smd roundrect (at -0.825 0 90) (size 0.8 0.95) (layers "F.Cu" "F.Mask" "F.Paste") (roundrect_rratio 0.25) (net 4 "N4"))
  (pad "2" smd roundrect (at 0.825 0 90) (size 0.8 0.95) (layers "F.Cu" "F.Mask" "F.Paste") (roundrect_rratio 0.25) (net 3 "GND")))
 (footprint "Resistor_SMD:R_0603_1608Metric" (layer "F.Cu") (at 159.25 97.758385)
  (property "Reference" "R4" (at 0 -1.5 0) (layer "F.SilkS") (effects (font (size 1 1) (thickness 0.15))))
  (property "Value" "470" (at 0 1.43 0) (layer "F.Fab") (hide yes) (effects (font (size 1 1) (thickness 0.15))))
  (fp_line (start -0.237258 -0.5225) (end 0.237258 -0.5225) (stroke (width 0.12) (type solid)) (layer "F.SilkS"))
  (fp_line (start -0.237258 0.5225) (end 0.237258 0.5225) (stroke (width 0.12) (type solid)) (layer "F.SilkS"))
  (pad "1" smd roundrect (at -0.825 0) (size 0.8 0.95) (layers "F.Cu" "F.Mask" "F.Paste") (roundrect_rratio 0.25) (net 8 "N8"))
  (pad "2" smd roundrect (at 0.825 0) (size 0.8 0.95) (layers "F.Cu" "F.Mask" "F.Paste") (roundrect_rratio 0.25) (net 9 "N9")))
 (gr_rect (start 147.85 95.25) (end 178.35 106.75) (stroke (width 0.05) (type default)) (fill no) (layer "Edge.Cuts"))
 (segment (start 156.275 101.275) (end 159 101.275) (width 0.2) (layer "F.Cu") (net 6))
 (segment (start 154.45 100) (end 155.45 101) (width 0.2) (layer "F.Cu") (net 6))
 (segment (start 155.45 101) (end 156 101) (width 0.2) (layer "F.Cu") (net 6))
 (segment (start 156 101) (end 156.275 101.275) (width 0.2) (layer "F.Cu") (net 6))
 (segment (start 159.775 101.275) (end 159.958385 101.458385) (width 0.2) (layer "F.Cu") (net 6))
 (segment (start 159 101.275) (end 159.775 101.275) (width 0.2) (layer "F.Cu") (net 6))
 (segment (start 159.958385 101.458385) (end 161.133495 101.458385) (width 0.2) (layer "F.Cu") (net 6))
 (segment (start 169.5 97.675) (end 167.5 97.675) (width 0.2) (layer "F.Cu") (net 3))
 (segment (start 161.133495 100.508385) (end 162.491615 100.508385) (width 0.2) (layer "F.Cu") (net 3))
 (segment (start 159.783385 100.508385) (end 161.133495 100.508385) (width 0.2) (layer "F.Cu") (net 3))
 (segment (start 154.45 102) (end 156 102) (width 0.2) (layer "F.Cu") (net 3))
 (segment (start 165.658385 97.675) (end 165.575 97.758385) (width 0.2) (layer "F.Cu") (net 3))
 (segment (start 164.725 100.5) (end 162.5 100.5) (width 0.2) (layer "F.Cu") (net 3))
 (segment (start 159 99.725) (end 159.783385 100.508385) (width 0.2) (layer "F.Cu") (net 3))
 (segment (start 172.75 103.75) (end 173 103.5) (width 0.2) (layer "F.Cu") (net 3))
 (segment (start 171.92 103.75) (end 172.75 103.75) (width 0.2) (layer "F.Cu") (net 3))
 (segment (start 167.5 97.675) (end 165.658385 97.675) (width 0.2) (layer "F.Cu") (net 3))
 (segment (start 162.491615 100.508385) (end 162.5 100.5) (width 0.2) (layer "F.Cu") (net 3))
 (segment (start 165.575 97.758385) (end 165.575 99.65) (width 0.2) (layer "F.Cu") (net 3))
 (segment (start 162.2125 105.5) (end 161 105.5) (width 0.2) (layer "F.Cu") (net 3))
 (segment (start 165.575 99.65) (end 165.5 99.725) (width 0.2) (layer "F.Cu") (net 3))
 (segment (start 171.92 98.25) (end 170.075 98.25) (width 0.2) (layer "F.Cu") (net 3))
 (segment (start 165.5 99.725) (end 164.725 100.5) (width 0.2) (layer "F.Cu") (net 3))
 (segment (start 170.075 98.25) (end 169.5 97.675) (width 0.2) (layer "F.Cu") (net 3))
 (via (at 162.5 100.5) (size 0.6) (drill 0.3) (layers "F.Cu" "B.Cu") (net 3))
 (via (at 173 103.5) (size 0.6) (drill 0.3) (layers "F.Cu" "B.Cu") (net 3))
 (via (at 156 102) (size 0.6) (drill 0.3) (layers "F.Cu" "B.Cu") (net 3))
 (via (at 161 105.5) (size 0.6) (drill 0.3) (layers "F.Cu" "B.Cu") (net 3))
 (segment (start 171.92 99.48) (end 172.52 99.48) (width 0.2) (layer "F.Cu") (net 2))
 (segment (start 171.48 102.52) (end 170.666356 103.333644) (width 0.2) (layer "F.Cu") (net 2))
 (segment (start 173 99.96) (end 173 102) (width 0.2) (layer "F.Cu") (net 2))
 (segment (start 171.92 102.52) (end 171.48 102.52) (width 0.2) (layer "F.Cu") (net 2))
 (segment (start 165.5 103.333644) (end 163.953856 103.333644) (width 0.2) (layer "F.Cu") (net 2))
 (segment (start 165.5 103.333644) (end 165.5 101.275) (width 0.2) (layer "F.Cu") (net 2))
 (segment (start 165.5 101.275) (end 163.59188 101.275) (width 0.2) (layer "F.Cu") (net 2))
 (segment (start 172.48 102.52) (end 171.92 102.52) (width 0.2) (layer "F.Cu") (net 2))
 (segment (start 172.52 99.48) (end 173 99.96) (width 0.2) (layer "F.Cu") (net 2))
 (segment (start 163.59188 101.275) (end 163.408495 101.458385) (width 0.2) (layer "F.Cu") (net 2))
 (segment (start 170.666356 103.333644) (end 165.5 103.333644) (width 0.2) (layer "F.Cu") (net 2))
 (segment (start 173 102) (end 172.48 102.52) (width 0.2) (layer "F.Cu") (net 2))
 (segment (start 163.953856 103.333644) (end 163.7875 103.5) (width 0.2) (layer "F.Cu") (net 2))
 (segment (start 157.5 98) (end 158.183385 98) (width 0.2) (layer "F.Cu") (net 8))
 (segment (start 157 98.5) (end 157.5 98) (width 0.2) (layer "F.Cu") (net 8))
 (segment (start 158.183385 98) (end 158.425 97.758385) (width 0.2) (layer "F.Cu") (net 8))
 (segment (start 162.2125 103.5) (end 161 103.5) (width 0.2) (layer "F.Cu") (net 8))
 (via (at 157 98.5) (size 0.6) (drill 0.3) (layers "F.Cu" "B.Cu") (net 8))
 (via (at 161 103.5) (size 0.6) (drill 0.3) (layers "F.Cu" "B.Cu") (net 8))
 (segment (start 157 99.5) (end 161 103.5) (width 0.2) (layer "B.Cu") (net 8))
 (segment (start 157 98.5) (end 157 99.5) (width 0.2) (layer "B.Cu") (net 8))
 (segment (start 165.5 104.983644) (end 164.303856 104.983644) (width 0.2) (layer "F.Cu") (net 10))
 (segment (start 164.303856 104.983644) (end 163.7875 105.5) (width 0.2) (layer "F.Cu") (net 10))
 (segment (start 175.8 105.32) (end 172 105.32) (width 0.2) (layer "F.Cu") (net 5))
 (segment (start 172 96.68) (end 175.8 96.68) (width 0.2) (layer "F.Cu") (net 5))
 (segment (start 175.8 96.68) (end 175.8 105.32) (width 0.2) (layer "F.Cu") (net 5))
 (segment (start 169.675 101.5) (end 167.5 99.325) (width 0.2) (layer "F.Cu") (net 1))
 (segment (start 171.92 101.5) (end 169.675 101.5) (width 0.2) (layer "F.Cu") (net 1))
 (segment (start 170.675 100.5) (end 171.92 100.5) (width 0.2) (layer "F.Cu") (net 4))
 (segment (start 169.5 99.325) (end 170.675 100.5) (width 0.2) (layer "F.Cu") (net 4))
 (segment (start 163.408495 99.558385) (end 163.925 99.04188) (width 0.2) (layer "F.Cu") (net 7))
 (segment (start 163.925 99.04188) (end 163.925 97.758385) (width 0.2) (layer "F.Cu") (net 7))
 (segment (start 160.075 98.49989) (end 161.133495 99.558385) (width 0.2) (layer "F.Cu") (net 9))
 (segment (start 160.075 97.758385) (end 160.075 98.49989) (width 0.2) (layer "F.Cu") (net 9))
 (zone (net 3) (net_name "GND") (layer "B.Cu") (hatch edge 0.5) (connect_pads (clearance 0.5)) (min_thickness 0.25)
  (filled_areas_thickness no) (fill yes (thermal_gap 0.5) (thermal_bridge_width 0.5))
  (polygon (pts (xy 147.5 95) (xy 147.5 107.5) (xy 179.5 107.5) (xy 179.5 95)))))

